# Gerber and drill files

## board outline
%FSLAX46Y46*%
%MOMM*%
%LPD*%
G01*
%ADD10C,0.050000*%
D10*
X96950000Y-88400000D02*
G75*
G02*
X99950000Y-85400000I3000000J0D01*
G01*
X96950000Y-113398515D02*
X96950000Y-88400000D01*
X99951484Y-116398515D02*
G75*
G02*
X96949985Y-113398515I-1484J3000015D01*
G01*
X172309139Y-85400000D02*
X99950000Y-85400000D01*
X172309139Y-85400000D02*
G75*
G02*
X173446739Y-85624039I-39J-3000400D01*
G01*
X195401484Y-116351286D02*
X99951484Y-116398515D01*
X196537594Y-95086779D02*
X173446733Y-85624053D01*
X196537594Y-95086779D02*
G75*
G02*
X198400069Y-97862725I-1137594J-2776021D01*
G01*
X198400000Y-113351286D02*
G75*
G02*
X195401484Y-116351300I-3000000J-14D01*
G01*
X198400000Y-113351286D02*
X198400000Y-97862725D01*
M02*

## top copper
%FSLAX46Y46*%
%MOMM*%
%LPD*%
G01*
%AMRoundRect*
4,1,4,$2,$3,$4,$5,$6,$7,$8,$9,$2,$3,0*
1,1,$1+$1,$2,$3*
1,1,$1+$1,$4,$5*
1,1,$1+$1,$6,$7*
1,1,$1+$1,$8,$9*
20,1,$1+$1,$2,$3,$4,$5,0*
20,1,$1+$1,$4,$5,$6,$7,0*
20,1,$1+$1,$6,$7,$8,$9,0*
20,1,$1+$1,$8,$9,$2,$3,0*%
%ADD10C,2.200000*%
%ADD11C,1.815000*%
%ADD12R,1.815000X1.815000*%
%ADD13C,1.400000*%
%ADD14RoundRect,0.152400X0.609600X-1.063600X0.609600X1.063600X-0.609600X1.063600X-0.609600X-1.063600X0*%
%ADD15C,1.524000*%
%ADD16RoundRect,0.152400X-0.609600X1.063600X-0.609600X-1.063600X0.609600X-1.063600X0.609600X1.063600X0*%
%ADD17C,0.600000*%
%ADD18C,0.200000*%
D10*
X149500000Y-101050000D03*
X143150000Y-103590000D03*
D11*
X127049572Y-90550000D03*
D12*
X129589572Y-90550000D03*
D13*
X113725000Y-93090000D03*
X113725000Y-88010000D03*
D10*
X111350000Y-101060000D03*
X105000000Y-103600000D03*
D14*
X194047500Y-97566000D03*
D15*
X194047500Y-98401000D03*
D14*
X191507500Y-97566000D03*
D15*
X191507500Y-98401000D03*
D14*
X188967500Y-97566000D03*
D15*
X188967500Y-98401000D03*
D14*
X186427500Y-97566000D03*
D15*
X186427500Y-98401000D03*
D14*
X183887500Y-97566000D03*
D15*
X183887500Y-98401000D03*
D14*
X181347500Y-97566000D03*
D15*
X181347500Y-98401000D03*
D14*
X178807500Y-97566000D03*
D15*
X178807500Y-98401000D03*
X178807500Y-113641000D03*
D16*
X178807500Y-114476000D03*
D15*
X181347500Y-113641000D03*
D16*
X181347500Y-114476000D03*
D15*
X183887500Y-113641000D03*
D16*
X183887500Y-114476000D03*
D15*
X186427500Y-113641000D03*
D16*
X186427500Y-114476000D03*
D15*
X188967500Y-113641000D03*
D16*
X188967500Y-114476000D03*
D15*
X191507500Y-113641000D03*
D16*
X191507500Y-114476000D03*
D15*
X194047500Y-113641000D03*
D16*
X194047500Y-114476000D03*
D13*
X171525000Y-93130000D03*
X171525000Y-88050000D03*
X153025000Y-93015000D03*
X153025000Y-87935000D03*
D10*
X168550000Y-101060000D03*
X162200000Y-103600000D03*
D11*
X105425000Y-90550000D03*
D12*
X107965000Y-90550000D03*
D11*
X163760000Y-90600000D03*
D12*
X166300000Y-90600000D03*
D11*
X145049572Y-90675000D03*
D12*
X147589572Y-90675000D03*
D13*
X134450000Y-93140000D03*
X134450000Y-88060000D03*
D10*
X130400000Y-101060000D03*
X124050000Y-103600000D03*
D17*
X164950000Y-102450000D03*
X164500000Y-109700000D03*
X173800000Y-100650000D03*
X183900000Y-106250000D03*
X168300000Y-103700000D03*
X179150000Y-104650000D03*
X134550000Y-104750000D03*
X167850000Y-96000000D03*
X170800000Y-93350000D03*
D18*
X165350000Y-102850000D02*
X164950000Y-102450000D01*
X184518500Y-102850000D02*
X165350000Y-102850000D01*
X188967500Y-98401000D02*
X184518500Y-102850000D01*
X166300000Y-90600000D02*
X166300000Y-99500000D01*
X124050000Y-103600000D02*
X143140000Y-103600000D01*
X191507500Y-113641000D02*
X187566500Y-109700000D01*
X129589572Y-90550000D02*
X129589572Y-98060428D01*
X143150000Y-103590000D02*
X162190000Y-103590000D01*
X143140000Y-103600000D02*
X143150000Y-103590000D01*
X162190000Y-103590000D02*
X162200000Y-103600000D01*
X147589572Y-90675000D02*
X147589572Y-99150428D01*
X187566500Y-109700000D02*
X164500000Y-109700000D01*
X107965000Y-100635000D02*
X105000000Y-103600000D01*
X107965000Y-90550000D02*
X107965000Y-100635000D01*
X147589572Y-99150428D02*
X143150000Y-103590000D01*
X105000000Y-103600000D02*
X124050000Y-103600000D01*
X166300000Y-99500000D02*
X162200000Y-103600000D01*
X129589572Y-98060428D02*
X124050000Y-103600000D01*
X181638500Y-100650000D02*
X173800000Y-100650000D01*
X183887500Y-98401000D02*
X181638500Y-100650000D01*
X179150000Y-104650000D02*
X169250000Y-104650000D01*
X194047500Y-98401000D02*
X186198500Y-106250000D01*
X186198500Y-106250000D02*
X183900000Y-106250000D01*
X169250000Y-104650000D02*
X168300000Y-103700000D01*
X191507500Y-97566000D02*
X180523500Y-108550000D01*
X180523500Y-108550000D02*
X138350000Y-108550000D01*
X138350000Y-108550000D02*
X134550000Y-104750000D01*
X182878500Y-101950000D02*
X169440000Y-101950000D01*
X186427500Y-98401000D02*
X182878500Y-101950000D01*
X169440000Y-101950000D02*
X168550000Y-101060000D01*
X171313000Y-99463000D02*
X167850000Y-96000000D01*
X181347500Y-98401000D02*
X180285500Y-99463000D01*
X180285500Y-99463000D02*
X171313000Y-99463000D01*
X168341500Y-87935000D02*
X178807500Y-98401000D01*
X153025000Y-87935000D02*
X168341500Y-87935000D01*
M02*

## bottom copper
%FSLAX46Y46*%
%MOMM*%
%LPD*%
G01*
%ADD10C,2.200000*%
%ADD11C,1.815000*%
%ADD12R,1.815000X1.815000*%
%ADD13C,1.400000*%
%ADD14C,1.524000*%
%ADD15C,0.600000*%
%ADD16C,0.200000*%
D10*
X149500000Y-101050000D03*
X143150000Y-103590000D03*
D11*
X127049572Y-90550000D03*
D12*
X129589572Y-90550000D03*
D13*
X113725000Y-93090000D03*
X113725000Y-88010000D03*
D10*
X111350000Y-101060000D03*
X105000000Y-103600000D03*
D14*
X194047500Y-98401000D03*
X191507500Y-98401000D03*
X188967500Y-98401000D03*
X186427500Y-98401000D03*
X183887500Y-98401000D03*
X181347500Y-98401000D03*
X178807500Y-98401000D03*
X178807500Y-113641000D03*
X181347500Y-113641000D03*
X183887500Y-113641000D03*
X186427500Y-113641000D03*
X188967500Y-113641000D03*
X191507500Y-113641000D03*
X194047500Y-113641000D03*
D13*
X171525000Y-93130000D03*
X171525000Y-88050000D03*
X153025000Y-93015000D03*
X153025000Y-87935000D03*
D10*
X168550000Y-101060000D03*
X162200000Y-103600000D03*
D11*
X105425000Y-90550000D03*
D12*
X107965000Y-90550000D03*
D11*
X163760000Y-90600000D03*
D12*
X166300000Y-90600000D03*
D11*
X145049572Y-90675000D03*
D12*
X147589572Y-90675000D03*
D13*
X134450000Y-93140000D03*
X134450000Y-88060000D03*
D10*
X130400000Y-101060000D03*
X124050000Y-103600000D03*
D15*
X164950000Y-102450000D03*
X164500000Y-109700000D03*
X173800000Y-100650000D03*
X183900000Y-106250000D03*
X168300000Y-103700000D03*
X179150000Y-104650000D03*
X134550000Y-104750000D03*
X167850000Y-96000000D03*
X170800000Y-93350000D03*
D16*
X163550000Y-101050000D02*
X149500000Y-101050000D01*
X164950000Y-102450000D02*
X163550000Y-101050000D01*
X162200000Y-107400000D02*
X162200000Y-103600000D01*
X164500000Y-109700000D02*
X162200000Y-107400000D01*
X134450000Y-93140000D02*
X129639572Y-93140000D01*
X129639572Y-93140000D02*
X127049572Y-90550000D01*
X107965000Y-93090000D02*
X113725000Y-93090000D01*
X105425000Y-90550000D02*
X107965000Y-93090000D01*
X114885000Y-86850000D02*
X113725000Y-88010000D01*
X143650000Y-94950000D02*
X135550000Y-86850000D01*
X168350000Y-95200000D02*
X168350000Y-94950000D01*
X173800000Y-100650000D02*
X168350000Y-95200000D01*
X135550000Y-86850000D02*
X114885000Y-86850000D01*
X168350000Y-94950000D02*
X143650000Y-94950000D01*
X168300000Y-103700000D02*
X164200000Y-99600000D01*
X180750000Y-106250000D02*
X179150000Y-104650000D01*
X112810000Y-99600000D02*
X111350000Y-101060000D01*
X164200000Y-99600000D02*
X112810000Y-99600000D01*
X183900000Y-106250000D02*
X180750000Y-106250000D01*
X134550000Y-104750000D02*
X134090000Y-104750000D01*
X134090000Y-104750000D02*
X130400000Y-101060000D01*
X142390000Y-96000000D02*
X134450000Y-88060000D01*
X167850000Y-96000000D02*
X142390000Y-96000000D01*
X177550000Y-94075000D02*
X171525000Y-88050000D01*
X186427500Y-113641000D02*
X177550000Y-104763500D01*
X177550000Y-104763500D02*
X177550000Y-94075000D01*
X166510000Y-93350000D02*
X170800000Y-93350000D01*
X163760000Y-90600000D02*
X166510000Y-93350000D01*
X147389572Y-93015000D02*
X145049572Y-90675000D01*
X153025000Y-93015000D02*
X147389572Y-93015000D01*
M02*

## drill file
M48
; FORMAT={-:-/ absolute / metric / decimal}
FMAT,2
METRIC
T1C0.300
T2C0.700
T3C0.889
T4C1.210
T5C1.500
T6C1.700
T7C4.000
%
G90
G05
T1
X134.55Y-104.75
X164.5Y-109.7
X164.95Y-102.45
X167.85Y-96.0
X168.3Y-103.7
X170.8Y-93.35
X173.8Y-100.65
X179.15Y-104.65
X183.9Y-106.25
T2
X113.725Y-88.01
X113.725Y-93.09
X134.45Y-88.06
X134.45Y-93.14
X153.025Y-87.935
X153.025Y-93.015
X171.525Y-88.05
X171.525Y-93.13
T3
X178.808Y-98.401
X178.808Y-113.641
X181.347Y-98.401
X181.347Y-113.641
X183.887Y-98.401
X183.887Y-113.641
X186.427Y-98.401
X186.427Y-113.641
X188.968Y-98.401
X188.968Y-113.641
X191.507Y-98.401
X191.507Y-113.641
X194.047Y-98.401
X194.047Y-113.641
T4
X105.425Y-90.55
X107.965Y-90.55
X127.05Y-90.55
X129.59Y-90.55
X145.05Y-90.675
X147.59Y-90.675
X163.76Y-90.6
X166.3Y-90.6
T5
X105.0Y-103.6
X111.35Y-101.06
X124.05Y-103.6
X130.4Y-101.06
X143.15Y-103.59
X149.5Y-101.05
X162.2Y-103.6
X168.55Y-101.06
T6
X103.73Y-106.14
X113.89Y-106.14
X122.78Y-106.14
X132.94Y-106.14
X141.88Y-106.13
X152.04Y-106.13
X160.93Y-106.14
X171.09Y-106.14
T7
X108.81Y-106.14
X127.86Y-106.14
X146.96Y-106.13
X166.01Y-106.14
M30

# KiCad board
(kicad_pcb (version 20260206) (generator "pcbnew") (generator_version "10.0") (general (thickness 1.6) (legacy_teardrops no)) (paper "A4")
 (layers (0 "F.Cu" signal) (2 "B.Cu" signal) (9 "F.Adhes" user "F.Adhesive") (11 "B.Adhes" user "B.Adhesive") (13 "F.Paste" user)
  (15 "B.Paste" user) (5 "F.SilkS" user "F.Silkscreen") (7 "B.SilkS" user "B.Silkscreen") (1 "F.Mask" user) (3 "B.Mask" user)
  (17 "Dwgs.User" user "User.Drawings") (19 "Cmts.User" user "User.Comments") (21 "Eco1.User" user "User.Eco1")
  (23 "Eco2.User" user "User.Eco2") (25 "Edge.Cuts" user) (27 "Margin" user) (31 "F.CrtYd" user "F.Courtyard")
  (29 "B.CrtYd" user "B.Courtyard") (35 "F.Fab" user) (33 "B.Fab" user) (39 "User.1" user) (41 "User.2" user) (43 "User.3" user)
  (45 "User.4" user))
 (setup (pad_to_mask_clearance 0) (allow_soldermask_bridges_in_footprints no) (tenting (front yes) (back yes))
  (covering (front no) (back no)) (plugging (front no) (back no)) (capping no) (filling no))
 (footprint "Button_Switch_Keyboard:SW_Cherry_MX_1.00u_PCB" (layer "F.Cu") (at 149.5 101.05)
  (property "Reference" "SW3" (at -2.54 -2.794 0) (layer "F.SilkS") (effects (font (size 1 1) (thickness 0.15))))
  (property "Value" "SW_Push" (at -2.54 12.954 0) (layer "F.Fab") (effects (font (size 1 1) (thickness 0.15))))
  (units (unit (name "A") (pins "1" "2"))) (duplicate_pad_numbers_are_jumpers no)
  (pad "" np_thru_hole circle (at -7.62 5.08) (size 1.7 1.7) (drill 1.7) (layers "*.Cu" "*.Mask"))
  (pad "" np_thru_hole circle (at -2.54 5.08) (size 4 4) (drill 4) (layers "*.Cu" "*.Mask"))
  (pad "" np_thru_hole circle (at 2.54 5.08) (size 1.7 1.7) (drill 1.7) (layers "*.Cu" "*.Mask"))
  (pad "1" thru_hole circle (at 0 0) (size 2.2 2.2) (drill 1.5) (layers "*.Cu" "*.Mask") (remove_unused_layers no) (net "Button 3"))
  (pad "2" thru_hole circle (at -6.35 2.54) (size 2.2 2.2) (drill 1.5) (layers "*.Cu" "*.Mask") (remove_unused_layers no) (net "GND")))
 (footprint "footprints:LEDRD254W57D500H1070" (layer "F.Cu") (at 128.319572 90.55 180)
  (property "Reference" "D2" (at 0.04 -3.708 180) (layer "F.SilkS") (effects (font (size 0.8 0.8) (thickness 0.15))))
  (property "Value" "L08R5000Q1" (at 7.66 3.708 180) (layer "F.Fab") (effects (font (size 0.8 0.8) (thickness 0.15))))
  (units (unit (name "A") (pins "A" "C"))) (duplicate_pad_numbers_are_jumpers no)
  (pad "A" thru_hole circle (at 1.27 0 180) (size 1.815 1.815) (drill 1.21) (layers "*.Cu" "*.Mask") (remove_unused_layers no)
   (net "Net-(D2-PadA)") (solder_mask_margin 0.102))
  (pad "C" thru_hole rect (at -1.27 0 180) (size 1.815 1.815) (drill 1.21) (layers "*.Cu" "*.Mask") (remove_unused_layers no) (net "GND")
   (solder_mask_margin 0.102)))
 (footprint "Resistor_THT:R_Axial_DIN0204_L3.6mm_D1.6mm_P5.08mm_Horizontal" (layer "F.Cu") (at 113.725 93.09 90)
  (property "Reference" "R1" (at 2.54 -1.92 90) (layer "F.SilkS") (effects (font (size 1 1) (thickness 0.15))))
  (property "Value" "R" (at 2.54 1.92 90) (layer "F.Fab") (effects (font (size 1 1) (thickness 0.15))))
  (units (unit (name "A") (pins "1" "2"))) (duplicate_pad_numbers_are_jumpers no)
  (pad "1" thru_hole circle (at 0 0 90) (size 1.4 1.4) (drill 0.7) (layers "*.Cu" "*.Mask") (remove_unused_layers no) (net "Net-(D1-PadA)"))
  (pad "2" thru_hole circle (at 5.08 0 90) (size 1.4 1.4) (drill 0.7) (layers "*.Cu" "*.Mask") (remove_unused_layers no) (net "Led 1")))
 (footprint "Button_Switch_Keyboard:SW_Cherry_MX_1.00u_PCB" (layer "F.Cu") (at 111.35 101.06)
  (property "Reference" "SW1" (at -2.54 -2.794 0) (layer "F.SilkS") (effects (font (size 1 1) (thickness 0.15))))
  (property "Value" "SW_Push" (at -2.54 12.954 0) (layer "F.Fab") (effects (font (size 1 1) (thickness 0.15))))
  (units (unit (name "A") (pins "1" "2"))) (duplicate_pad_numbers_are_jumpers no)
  (pad "" np_thru_hole circle (at -7.62 5.08) (size 1.7 1.7) (drill 1.7) (layers "*.Cu" "*.Mask"))
  (pad "" np_thru_hole circle (at -2.54 5.08) (size 4 4) (drill 4) (layers "*.Cu" "*.Mask"))
  (pad "" np_thru_hole circle (at 2.54 5.08) (size 1.7 1.7) (drill 1.7) (layers "*.Cu" "*.Mask"))
  (pad "1" thru_hole circle (at 0 0) (size 2.2 2.2) (drill 1.5) (layers "*.Cu" "*.Mask") (remove_unused_layers no) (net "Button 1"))
  (pad "2" thru_hole circle (at -6.35 2.54) (size 2.2 2.2) (drill 1.5) (layers "*.Cu" "*.Mask") (remove_unused_layers no) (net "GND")))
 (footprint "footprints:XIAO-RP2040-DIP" (layer "F.Cu") (at 186.4275 106.021)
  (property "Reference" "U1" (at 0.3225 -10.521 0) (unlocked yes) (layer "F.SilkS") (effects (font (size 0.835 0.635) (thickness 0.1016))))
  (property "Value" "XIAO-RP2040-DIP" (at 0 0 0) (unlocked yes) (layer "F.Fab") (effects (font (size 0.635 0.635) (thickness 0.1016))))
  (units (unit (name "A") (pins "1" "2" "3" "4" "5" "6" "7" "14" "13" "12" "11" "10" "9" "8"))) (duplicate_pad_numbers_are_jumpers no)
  (pad "1" smd roundrect (at 7.62 -8.455 90) (size 2.432 1.524) (layers "F.Cu" "F.Mask") (roundrect_rratio 0.1) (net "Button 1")
   (thermal_bridge_angle 45))
  (pad "1" thru_hole circle (at 7.62 -7.62 90) (size 1.524 1.524) (drill 0.889) (layers "*.Cu" "*.Mask") (remove_unused_layers no)
   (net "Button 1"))
  (pad "2" smd roundrect (at 5.08 -8.455 90) (size 2.432 1.524) (layers "F.Cu" "F.Mask") (roundrect_rratio 0.1) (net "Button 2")
   (thermal_bridge_angle 45))
  (pad "2" thru_hole circle (at 5.08 -7.62 90) (size 1.524 1.524) (drill 0.889) (layers "*.Cu" "*.Mask") (remove_unused_layers no)
   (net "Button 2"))
  (pad "3" smd roundrect (at 2.54 -8.455 90) (size 2.432 1.524) (layers "F.Cu" "F.Mask") (roundrect_rratio 0.1) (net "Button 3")
   (thermal_bridge_angle 45))
  (pad "3" thru_hole circle (at 2.54 -7.62 90) (size 1.524 1.524) (drill 0.889) (layers "*.Cu" "*.Mask") (remove_unused_layers no)
   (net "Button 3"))
  (pad "4" smd roundrect (at 0 -8.455 90) (size 2.432 1.524) (layers "F.Cu" "F.Mask") (roundrect_rratio 0.1) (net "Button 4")
   (thermal_bridge_angle 45))
  (pad "4" thru_hole circle (at 0 -7.62 90) (size 1.524 1.524) (drill 0.889) (layers "*.Cu" "*.Mask") (remove_unused_layers no)
   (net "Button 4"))
  (pad "5" smd roundrect (at -2.54 -8.455 90) (size 2.432 1.524) (layers "F.Cu" "F.Mask") (roundrect_rratio 0.1) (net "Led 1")
   (thermal_bridge_angle 45))
  (pad "5" thru_hole circle (at -2.54 -7.62 90) (size 1.524 1.524) (drill 0.889) (layers "*.Cu" "*.Mask") (remove_unused_layers no)
   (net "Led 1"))
  (pad "6" smd roundrect (at -5.08 -8.455 90) (size 2.432 1.524) (layers "F.Cu" "F.Mask") (roundrect_rratio 0.1) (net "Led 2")
   (thermal_bridge_angle 45))
  (pad "6" thru_hole circle (at -5.08 -7.62 90) (size 1.524 1.524) (drill 0.889) (layers "*.Cu" "*.Mask") (remove_unused_layers no)
   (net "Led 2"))
  (pad "7" smd roundrect (at -7.62 -8.455 90) (size 2.432 1.524) (layers "F.Cu" "F.Mask") (roundrect_rratio 0.1) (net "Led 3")
   (thermal_bridge_angle 45))
  (pad "7" thru_hole circle (at -7.62 -7.62 90) (size 1.524 1.524) (drill 0.889) (layers "*.Cu" "*.Mask") (remove_unused_layers no)
   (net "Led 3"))
  (pad "8" thru_hole circle (at -7.62 7.62 270) (size 1.524 1.524) (drill 0.889) (layers "*.Cu" "*.Mask") (remove_unused_layers no)
   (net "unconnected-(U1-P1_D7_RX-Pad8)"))
  (pad "8" smd roundrect (at -7.62 8.455 270) (size 2.432 1.524) (layers "F.Cu" "F.Mask") (roundrect_rratio 0.1)
   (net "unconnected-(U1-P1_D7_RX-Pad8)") (thermal_bridge_angle 45))
  (pad "9" thru_hole circle (at -5.08 7.62 270) (size 1.524 1.524) (drill 0.889) (layers "*.Cu" "*.Mask") (remove_unused_layers no)
   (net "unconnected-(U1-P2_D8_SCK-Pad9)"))
  (pad "9" smd roundrect (at -5.08 8.455 270) (size 2.432 1.524) (layers "F.Cu" "F.Mask") (roundrect_rratio 0.1)
   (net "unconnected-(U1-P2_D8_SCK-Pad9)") (thermal_bridge_angle 45))
  (pad "10" thru_hole circle (at -2.54 7.62 270) (size 1.524 1.524) (drill 0.889) (layers "*.Cu" "*.Mask") (remove_unused_layers no)
   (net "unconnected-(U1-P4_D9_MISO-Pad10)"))
  (pad "10" smd roundrect (at -2.54 8.455 270) (size 2.432 1.524) (layers "F.Cu" "F.Mask") (roundrect_rratio 0.1)
   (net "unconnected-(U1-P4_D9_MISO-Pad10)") (thermal_bridge_angle 45))
  (pad "11" thru_hole circle (at 0 7.62 270) (size 1.524 1.524) (drill 0.889) (layers "*.Cu" "*.Mask") (remove_unused_layers no)
   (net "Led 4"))
  (pad "11" smd roundrect (at 0 8.455 270) (size 2.432 1.524) (layers "F.Cu" "F.Mask") (roundrect_rratio 0.1) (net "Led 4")
   (thermal_bridge_angle 45))
  (pad "12" thru_hole circle (at 2.54 7.62 270) (size 1.524 1.524) (drill 0.889) (layers "*.Cu" "*.Mask") (remove_unused_layers no)
   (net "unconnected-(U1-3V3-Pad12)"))
  (pad "12" smd roundrect (at 2.54 8.455 270) (size 2.432 1.524) (layers "F.Cu" "F.Mask") (roundrect_rratio 0.1)
   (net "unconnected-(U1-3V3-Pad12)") (thermal_bridge_angle 45))
  (pad "13" thru_hole circle (at 5.08 7.62 270) (size 1.524 1.524) (drill 0.889) (layers "*.Cu" "*.Mask") (remove_unused_layers no)
   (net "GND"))
  (pad "13" smd roundrect (at 5.08 8.455 270) (size 2.432 1.524) (layers "F.Cu" "F.Mask") (roundrect_rratio 0.1) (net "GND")
   (thermal_bridge_angle 45))
  (pad "14" thru_hole circle (at 7.62 7.62 270) (size 1.524 1.524) (drill 0.889) (layers "*.Cu" "*.Mask") (remove_unused_layers no)
   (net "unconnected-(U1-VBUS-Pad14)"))
  (pad "14" smd roundrect (at 7.62 8.455 270) (size 2.432 1.524) (layers "F.Cu" "F.Mask") (roundrect_rratio 0.1)
   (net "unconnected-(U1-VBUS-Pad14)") (thermal_bridge_angle 45)))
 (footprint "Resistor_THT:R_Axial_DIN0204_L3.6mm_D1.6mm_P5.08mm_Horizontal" (layer "F.Cu") (at 171.525 93.13 90)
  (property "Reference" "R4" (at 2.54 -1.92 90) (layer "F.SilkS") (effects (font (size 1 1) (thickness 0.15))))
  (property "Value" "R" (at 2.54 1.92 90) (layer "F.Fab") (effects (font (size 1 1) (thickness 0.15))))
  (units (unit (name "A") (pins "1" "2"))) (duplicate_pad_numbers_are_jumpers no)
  (pad "1" thru_hole circle (at 0 0 90) (size 1.4 1.4) (drill 0.7) (layers "*.Cu" "*.Mask") (remove_unused_layers no) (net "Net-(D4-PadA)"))
  (pad "2" thru_hole circle (at 5.08 0 90) (size 1.4 1.4) (drill 0.7) (layers "*.Cu" "*.Mask") (remove_unused_layers no) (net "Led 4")))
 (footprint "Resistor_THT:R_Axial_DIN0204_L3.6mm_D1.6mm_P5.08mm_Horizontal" (layer "F.Cu") (at 153.025 93.015 90)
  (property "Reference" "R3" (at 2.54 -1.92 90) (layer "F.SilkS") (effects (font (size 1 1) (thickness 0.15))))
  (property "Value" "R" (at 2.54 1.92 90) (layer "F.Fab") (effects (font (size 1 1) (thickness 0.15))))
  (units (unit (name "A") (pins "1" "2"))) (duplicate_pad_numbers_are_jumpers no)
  (pad "1" thru_hole circle (at 0 0 90) (size 1.4 1.4) (drill 0.7) (layers "*.Cu" "*.Mask") (remove_unused_layers no) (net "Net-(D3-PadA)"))
  (pad "2" thru_hole circle (at 5.08 0 90) (size 1.4 1.4) (drill 0.7) (layers "*.Cu" "*.Mask") (remove_unused_layers no) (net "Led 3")))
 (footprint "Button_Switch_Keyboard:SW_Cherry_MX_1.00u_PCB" (layer "F.Cu") (at 168.55 101.06)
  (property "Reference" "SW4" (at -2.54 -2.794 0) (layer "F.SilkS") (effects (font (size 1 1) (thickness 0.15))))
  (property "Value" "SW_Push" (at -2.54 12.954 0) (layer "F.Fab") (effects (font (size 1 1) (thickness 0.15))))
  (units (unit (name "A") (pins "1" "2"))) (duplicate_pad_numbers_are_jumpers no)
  (pad "" np_thru_hole circle (at -7.62 5.08) (size 1.7 1.7) (drill 1.7) (layers "*.Cu" "*.Mask"))
  (pad "" np_thru_hole circle (at -2.54 5.08) (size 4 4) (drill 4) (layers "*.Cu" "*.Mask"))
  (pad "" np_thru_hole circle (at 2.54 5.08) (size 1.7 1.7) (drill 1.7) (layers "*.Cu" "*.Mask"))
  (pad "1" thru_hole circle (at 0 0) (size 2.2 2.2) (drill 1.5) (layers "*.Cu" "*.Mask") (remove_unused_layers no) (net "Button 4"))
  (pad "2" thru_hole circle (at -6.35 2.54) (size 2.2 2.2) (drill 1.5) (layers "*.Cu" "*.Mask") (remove_unused_layers no) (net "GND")))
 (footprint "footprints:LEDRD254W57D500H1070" (layer "F.Cu") (at 106.695 90.55 180)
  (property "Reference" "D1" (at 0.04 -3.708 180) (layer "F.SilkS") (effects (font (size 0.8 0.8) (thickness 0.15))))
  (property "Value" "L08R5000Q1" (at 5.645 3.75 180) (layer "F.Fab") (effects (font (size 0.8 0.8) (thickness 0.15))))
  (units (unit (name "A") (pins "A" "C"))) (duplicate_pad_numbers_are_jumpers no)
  (pad "A" thru_hole circle (at 1.27 0 180) (size 1.815 1.815) (drill 1.21) (layers "*.Cu" "*.Mask") (remove_unused_layers no)
   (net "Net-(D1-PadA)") (solder_mask_margin 0.102))
  (pad "C" thru_hole rect (at -1.27 0 180) (size 1.815 1.815) (drill 1.21) (layers "*.Cu" "*.Mask") (remove_unused_layers no) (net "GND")
   (solder_mask_margin 0.102)))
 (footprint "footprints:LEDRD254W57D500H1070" (layer "F.Cu") (at 165.03 90.6 180)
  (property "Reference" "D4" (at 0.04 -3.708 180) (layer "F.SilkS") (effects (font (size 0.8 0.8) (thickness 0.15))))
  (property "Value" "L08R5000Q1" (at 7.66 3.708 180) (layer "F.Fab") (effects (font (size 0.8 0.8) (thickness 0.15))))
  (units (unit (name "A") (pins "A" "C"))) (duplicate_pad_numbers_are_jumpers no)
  (pad "A" thru_hole circle (at 1.27 0 180) (size 1.815 1.815) (drill 1.21) (layers "*.Cu" "*.Mask") (remove_unused_layers no)
   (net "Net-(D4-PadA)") (solder_mask_margin 0.102))
  (pad "C" thru_hole rect (at -1.27 0 180) (size 1.815 1.815) (drill 1.21) (layers "*.Cu" "*.Mask") (remove_unused_layers no) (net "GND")
   (solder_mask_margin 0.102)))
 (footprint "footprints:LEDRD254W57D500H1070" (layer "F.Cu") (at 146.319572 90.675 180)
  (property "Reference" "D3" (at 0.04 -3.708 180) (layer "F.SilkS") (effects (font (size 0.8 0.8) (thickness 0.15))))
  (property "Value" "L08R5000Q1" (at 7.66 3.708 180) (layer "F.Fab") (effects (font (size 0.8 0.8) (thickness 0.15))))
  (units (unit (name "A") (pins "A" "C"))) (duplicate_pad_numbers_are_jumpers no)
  (pad "A" thru_hole circle (at 1.27 0 180) (size 1.815 1.815) (drill 1.21) (layers "*.Cu" "*.Mask") (remove_unused_layers no)
   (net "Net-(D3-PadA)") (solder_mask_margin 0.102))
  (pad "C" thru_hole rect (at -1.27 0 180) (size 1.815 1.815) (drill 1.21) (layers "*.Cu" "*.Mask") (remove_unused_layers no) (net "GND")
   (solder_mask_margin 0.102)))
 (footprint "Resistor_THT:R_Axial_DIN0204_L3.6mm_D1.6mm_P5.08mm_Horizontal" (layer "F.Cu") (at 134.45 93.14 90)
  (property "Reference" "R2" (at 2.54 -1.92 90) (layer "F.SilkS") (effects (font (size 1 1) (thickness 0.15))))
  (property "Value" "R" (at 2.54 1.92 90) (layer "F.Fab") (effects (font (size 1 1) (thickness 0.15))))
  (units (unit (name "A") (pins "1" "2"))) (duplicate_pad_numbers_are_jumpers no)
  (pad "1" thru_hole circle (at 0 0 90) (size 1.4 1.4) (drill 0.7) (layers "*.Cu" "*.Mask") (remove_unused_layers no) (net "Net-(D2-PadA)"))
  (pad "2" thru_hole circle (at 5.08 0 90) (size 1.4 1.4) (drill 0.7) (layers "*.Cu" "*.Mask") (remove_unused_layers no) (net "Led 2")))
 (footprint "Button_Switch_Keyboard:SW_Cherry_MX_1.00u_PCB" (layer "F.Cu") (at 130.4 101.06)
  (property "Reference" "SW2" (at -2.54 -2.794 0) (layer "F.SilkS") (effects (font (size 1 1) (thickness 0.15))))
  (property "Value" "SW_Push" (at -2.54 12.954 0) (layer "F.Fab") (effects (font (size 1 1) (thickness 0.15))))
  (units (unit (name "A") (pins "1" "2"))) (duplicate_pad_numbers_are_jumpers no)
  (pad "" np_thru_hole circle (at -7.62 5.08) (size 1.7 1.7) (drill 1.7) (layers "*.Cu" "*.Mask"))
  (pad "" np_thru_hole circle (at -2.54 5.08) (size 4 4) (drill 4) (layers "*.Cu" "*.Mask"))
  (pad "" np_thru_hole circle (at 2.54 5.08) (size 1.7 1.7) (drill 1.7) (layers "*.Cu" "*.Mask"))
  (pad "1" thru_hole circle (at 0 0) (size 2.2 2.2) (drill 1.5) (layers "*.Cu" "*.Mask") (remove_unused_layers no) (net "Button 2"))
  (pad "2" thru_hole circle (at -6.35 2.54) (size 2.2 2.2) (drill 1.5) (layers "*.Cu" "*.Mask") (remove_unused_layers no) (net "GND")))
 (gr_arc (start 96.95 88.4) (mid 97.82868 86.27868) (end 99.95 85.4) (stroke (width 0.05) (type default)) (layer "Edge.Cuts"))
 (gr_line (start 96.95 113.398515) (end 96.95 88.4) (stroke (width 0.05) (type default)) (layer "Edge.Cuts"))
 (gr_arc (start 99.951484 116.398515) (mid 97.829204 115.52036) (end 96.95 113.398515) (stroke (width 0.05) (type default))
  (layer "Edge.Cuts"))
 (gr_line (start 172.309139 85.4) (end 99.95 85.4) (stroke (width 0.05) (type default)) (layer "Edge.Cuts"))
 (gr_arc (start 172.309139 85.4) (mid 172.888861 85.456553) (end 173.446733 85.624053) (stroke (width 0.05) (type default))
  (layer "Edge.Cuts"))
 (gr_line (start 195.401484 116.351286) (end 99.951484 116.398515) (stroke (width 0.05) (type default)) (layer "Edge.Cuts"))
 (gr_line (start 196.537594 95.086779) (end 173.446733 85.624053) (stroke (width 0.05) (type default)) (layer "Edge.Cuts"))
 (gr_arc (start 196.537594 95.086779) (mid 197.891253 96.191318) (end 198.4 97.862725) (stroke (width 0.05) (type default))
  (layer "Edge.Cuts"))
 (gr_arc (start 198.4 113.351286) (mid 197.521845 115.472082) (end 195.401484 116.351286) (stroke (width 0.05) (type default))
  (layer "Edge.Cuts"))
 (gr_line (start 198.4 113.351286) (end 198.4 97.862725) (stroke (width 0.05) (type default)) (layer "Edge.Cuts"))
 (segment (start 165.35 102.85) (end 164.95 102.45) (width 0.2) (layer "F.Cu") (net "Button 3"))
 (segment (start 184.5185 102.85) (end 165.35 102.85) (width 0.2) (layer "F.Cu") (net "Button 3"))
 (segment (start 188.9675 98.401) (end 184.5185 102.85) (width 0.2) (layer "F.Cu") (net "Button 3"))
 (via (at 164.95 102.45) (size 0.6) (drill 0.3) (layers "F.Cu" "B.Cu") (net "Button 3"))
 (segment (start 163.55 101.05) (end 149.5 101.05) (width 0.2) (layer "B.Cu") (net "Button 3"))
 (segment (start 164.95 102.45) (end 163.55 101.05) (width 0.2) (layer "B.Cu") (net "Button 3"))
 (segment (start 166.3 90.6) (end 166.3 99.5) (width 0.2) (layer "F.Cu") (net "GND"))
 (segment (start 124.05 103.6) (end 143.14 103.6) (width 0.2) (layer "F.Cu") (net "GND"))
 (segment (start 191.5075 113.641) (end 187.5665 109.7) (width 0.2) (layer "F.Cu") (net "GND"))
 (segment (start 129.589572 90.55) (end 129.589572 98.060428) (width 0.2) (layer "F.Cu") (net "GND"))
 (segment (start 143.15 103.59) (end 162.19 103.59) (width 0.2) (layer "F.Cu") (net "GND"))
 (segment (start 143.14 103.6) (end 143.15 103.59) (width 0.2) (layer "F.Cu") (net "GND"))
 (segment (start 162.19 103.59) (end 162.2 103.6) (width 0.2) (layer "F.Cu") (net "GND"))
 (segment (start 147.589572 90.675) (end 147.589572 99.150428) (width 0.2) (layer "F.Cu") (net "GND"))
 (segment (start 187.5665 109.7) (end 164.5 109.7) (width 0.2) (layer "F.Cu") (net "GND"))
 (segment (start 107.965 100.635) (end 105 103.6) (width 0.2) (layer "F.Cu") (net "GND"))
 (segment (start 107.965 90.55) (end 107.965 100.635) (width 0.2) (layer "F.Cu") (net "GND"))
 (segment (start 147.589572 99.150428) (end 143.15 103.59) (width 0.2) (layer "F.Cu") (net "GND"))
 (segment (start 105 103.6) (end 124.05 103.6) (width 0.2) (layer "F.Cu") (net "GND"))
 (segment (start 166.3 99.5) (end 162.2 103.6) (width 0.2) (layer "F.Cu") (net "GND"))
 (segment (start 129.589572 98.060428) (end 124.05 103.6) (width 0.2) (layer "F.Cu") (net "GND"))
 (via (at 164.5 109.7) (size 0.6) (drill 0.3) (layers "F.Cu" "B.Cu") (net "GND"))
 (segment (start 162.2 107.4) (end 162.2 103.6) (width 0.2) (layer "B.Cu") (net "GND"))
 (segment (start 164.5 109.7) (end 162.2 107.4) (width 0.2) (layer "B.Cu") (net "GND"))
 (segment (start 134.45 93.14) (end 129.639572 93.14) (width 0.2) (layer "B.Cu") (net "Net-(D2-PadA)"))
 (segment (start 129.639572 93.14) (end 127.049572 90.55) (width 0.2) (layer "B.Cu") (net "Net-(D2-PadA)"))
 (segment (start 107.965 93.09) (end 113.725 93.09) (width 0.2) (layer "B.Cu") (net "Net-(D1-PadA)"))
 (segment (start 105.425 90.55) (end 107.965 93.09) (width 0.2) (layer "B.Cu") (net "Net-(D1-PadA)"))
 (segment (start 181.6385 100.65) (end 173.8 100.65) (width 0.2) (layer "F.Cu") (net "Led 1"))
 (segment (start 183.8875 98.401) (end 181.6385 100.65) (width 0.2) (layer "F.Cu") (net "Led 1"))
 (via (at 173.8 100.65) (size 0.6) (drill 0.3) (layers "F.Cu" "B.Cu") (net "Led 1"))
 (segment (start 114.885 86.85) (end 113.725 88.01) (width 0.2) (layer "B.Cu") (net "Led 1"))
 (segment (start 143.65 94.95) (end 135.55 86.85) (width 0.2) (layer "B.Cu") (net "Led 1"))
 (segment (start 168.35 95.2) (end 168.35 94.95) (width 0.2) (layer "B.Cu") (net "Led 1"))
 (segment (start 173.8 100.65) (end 168.35 95.2) (width 0.2) (layer "B.Cu") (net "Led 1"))
 (segment (start 135.55 86.85) (end 114.885 86.85) (width 0.2) (layer "B.Cu") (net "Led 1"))
 (segment (start 168.35 94.95) (end 143.65 94.95) (width 0.2) (layer "B.Cu") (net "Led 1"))
 (segment (start 179.15 104.65) (end 169.25 104.65) (width 0.2) (layer "F.Cu") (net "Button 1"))
 (segment (start 194.0475 98.401) (end 186.1985 106.25) (width 0.2) (layer "F.Cu") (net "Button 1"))
 (segment (start 186.1985 106.25) (end 183.9 106.25) (width 0.2) (layer "F.Cu") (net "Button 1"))
 (segment (start 169.25 104.65) (end 168.3 103.7) (width 0.2) (layer "F.Cu") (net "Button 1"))
 (via (at 183.9 106.25) (size 0.6) (drill 0.3) (layers "F.Cu" "B.Cu") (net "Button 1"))
 (via (at 168.3 103.7) (size 0.6) (drill 0.3) (layers "F.Cu" "B.Cu") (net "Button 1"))
 (via (at 179.15 104.65) (size 0.6) (drill 0.3) (layers "F.Cu" "B.Cu") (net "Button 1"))
 (segment (start 168.3 103.7) (end 164.2 99.6) (width 0.2) (layer "B.Cu") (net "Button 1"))
 (segment (start 180.75 106.25) (end 179.15 104.65) (width 0.2) (layer "B.Cu") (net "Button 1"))
 (segment (start 112.81 99.6) (end 111.35 101.06) (width 0.2) (layer "B.Cu") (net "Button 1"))
 (segment (start 164.2 99.6) (end 112.81 99.6) (width 0.2) (layer "B.Cu") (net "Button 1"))
 (segment (start 183.9 106.25) (end 180.75 106.25) (width 0.2) (layer "B.Cu") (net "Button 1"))
 (segment (start 191.5075 97.566) (end 180.5235 108.55) (width 0.2) (layer "F.Cu") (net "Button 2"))
 (segment (start 180.5235 108.55) (end 138.35 108.55) (width 0.2) (layer "F.Cu") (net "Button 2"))
 (segment (start 138.35 108.55) (end 134.55 104.75) (width 0.2) (layer "F.Cu") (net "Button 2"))
 (via (at 134.55 104.75) (size 0.6) (drill 0.3) (layers "F.Cu" "B.Cu") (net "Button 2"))
 (segment (start 134.55 104.75) (end 134.09 104.75) (width 0.2) (layer "B.Cu") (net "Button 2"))
 (segment (start 134.09 104.75) (end 130.4 101.06) (width 0.2) (layer "B.Cu") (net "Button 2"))
 (segment (start 182.8785 101.95) (end 169.44 101.95) (width 0.2) (layer "F.Cu") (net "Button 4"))
 (segment (start 186.4275 98.401) (end 182.8785 101.95) (width 0.2) (layer "F.Cu") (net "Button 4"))
 (segment (start 169.44 101.95) (end 168.55 101.06) (width 0.2) (layer "F.Cu") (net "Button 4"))
 (segment (start 171.313 99.463) (end 167.85 96) (width 0.2) (layer "F.Cu") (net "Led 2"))
 (segment (start 181.3475 98.401) (end 180.2855 99.463) (width 0.2) (layer "F.Cu") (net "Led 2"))
 (segment (start 180.2855 99.463) (end 171.313 99.463) (width 0.2) (layer "F.Cu") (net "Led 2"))
 (via (at 167.85 96) (size 0.6) (drill 0.3) (layers "F.Cu" "B.Cu") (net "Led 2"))
 (segment (start 142.39 96) (end 134.45 88.06) (width 0.2) (layer "B.Cu") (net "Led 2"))
 (segment (start 167.85 96) (end 142.39 96) (width 0.2) (layer "B.Cu") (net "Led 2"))
 (segment (start 168.3415 87.935) (end 178.8075 98.401) (width 0.2) (layer "F.Cu") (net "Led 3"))
 (segment (start 153.025 87.935) (end 168.3415 87.935) (width 0.2) (layer "F.Cu") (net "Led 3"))
 (segment (start 177.55 94.075) (end 171.525 88.05) (width 0.2) (layer "B.Cu") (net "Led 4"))
 (segment (start 186.4275 113.641) (end 177.55 104.7635) (width 0.2) (layer "B.Cu") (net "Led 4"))
 (segment (start 177.55 104.7635) (end 177.55 94.075) (width 0.2) (layer "B.Cu") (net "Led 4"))
 (via (at 170.8 93.35) (size 0.6) (drill 0.3) (layers "F.Cu" "B.Cu") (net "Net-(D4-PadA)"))
 (segment (start 166.51 93.35) (end 170.8 93.35) (width 0.2) (layer "B.Cu") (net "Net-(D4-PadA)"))
 (segment (start 163.76 90.6) (end 166.51 93.35) (width 0.2) (layer "B.Cu") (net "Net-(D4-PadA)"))
 (segment (start 147.389572 93.015) (end 145.049572 90.675) (width 0.2) (layer "B.Cu") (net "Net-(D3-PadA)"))
 (segment (start 153.025 93.015) (end 147.389572 93.015) (width 0.2) (layer "B.Cu") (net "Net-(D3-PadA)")))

